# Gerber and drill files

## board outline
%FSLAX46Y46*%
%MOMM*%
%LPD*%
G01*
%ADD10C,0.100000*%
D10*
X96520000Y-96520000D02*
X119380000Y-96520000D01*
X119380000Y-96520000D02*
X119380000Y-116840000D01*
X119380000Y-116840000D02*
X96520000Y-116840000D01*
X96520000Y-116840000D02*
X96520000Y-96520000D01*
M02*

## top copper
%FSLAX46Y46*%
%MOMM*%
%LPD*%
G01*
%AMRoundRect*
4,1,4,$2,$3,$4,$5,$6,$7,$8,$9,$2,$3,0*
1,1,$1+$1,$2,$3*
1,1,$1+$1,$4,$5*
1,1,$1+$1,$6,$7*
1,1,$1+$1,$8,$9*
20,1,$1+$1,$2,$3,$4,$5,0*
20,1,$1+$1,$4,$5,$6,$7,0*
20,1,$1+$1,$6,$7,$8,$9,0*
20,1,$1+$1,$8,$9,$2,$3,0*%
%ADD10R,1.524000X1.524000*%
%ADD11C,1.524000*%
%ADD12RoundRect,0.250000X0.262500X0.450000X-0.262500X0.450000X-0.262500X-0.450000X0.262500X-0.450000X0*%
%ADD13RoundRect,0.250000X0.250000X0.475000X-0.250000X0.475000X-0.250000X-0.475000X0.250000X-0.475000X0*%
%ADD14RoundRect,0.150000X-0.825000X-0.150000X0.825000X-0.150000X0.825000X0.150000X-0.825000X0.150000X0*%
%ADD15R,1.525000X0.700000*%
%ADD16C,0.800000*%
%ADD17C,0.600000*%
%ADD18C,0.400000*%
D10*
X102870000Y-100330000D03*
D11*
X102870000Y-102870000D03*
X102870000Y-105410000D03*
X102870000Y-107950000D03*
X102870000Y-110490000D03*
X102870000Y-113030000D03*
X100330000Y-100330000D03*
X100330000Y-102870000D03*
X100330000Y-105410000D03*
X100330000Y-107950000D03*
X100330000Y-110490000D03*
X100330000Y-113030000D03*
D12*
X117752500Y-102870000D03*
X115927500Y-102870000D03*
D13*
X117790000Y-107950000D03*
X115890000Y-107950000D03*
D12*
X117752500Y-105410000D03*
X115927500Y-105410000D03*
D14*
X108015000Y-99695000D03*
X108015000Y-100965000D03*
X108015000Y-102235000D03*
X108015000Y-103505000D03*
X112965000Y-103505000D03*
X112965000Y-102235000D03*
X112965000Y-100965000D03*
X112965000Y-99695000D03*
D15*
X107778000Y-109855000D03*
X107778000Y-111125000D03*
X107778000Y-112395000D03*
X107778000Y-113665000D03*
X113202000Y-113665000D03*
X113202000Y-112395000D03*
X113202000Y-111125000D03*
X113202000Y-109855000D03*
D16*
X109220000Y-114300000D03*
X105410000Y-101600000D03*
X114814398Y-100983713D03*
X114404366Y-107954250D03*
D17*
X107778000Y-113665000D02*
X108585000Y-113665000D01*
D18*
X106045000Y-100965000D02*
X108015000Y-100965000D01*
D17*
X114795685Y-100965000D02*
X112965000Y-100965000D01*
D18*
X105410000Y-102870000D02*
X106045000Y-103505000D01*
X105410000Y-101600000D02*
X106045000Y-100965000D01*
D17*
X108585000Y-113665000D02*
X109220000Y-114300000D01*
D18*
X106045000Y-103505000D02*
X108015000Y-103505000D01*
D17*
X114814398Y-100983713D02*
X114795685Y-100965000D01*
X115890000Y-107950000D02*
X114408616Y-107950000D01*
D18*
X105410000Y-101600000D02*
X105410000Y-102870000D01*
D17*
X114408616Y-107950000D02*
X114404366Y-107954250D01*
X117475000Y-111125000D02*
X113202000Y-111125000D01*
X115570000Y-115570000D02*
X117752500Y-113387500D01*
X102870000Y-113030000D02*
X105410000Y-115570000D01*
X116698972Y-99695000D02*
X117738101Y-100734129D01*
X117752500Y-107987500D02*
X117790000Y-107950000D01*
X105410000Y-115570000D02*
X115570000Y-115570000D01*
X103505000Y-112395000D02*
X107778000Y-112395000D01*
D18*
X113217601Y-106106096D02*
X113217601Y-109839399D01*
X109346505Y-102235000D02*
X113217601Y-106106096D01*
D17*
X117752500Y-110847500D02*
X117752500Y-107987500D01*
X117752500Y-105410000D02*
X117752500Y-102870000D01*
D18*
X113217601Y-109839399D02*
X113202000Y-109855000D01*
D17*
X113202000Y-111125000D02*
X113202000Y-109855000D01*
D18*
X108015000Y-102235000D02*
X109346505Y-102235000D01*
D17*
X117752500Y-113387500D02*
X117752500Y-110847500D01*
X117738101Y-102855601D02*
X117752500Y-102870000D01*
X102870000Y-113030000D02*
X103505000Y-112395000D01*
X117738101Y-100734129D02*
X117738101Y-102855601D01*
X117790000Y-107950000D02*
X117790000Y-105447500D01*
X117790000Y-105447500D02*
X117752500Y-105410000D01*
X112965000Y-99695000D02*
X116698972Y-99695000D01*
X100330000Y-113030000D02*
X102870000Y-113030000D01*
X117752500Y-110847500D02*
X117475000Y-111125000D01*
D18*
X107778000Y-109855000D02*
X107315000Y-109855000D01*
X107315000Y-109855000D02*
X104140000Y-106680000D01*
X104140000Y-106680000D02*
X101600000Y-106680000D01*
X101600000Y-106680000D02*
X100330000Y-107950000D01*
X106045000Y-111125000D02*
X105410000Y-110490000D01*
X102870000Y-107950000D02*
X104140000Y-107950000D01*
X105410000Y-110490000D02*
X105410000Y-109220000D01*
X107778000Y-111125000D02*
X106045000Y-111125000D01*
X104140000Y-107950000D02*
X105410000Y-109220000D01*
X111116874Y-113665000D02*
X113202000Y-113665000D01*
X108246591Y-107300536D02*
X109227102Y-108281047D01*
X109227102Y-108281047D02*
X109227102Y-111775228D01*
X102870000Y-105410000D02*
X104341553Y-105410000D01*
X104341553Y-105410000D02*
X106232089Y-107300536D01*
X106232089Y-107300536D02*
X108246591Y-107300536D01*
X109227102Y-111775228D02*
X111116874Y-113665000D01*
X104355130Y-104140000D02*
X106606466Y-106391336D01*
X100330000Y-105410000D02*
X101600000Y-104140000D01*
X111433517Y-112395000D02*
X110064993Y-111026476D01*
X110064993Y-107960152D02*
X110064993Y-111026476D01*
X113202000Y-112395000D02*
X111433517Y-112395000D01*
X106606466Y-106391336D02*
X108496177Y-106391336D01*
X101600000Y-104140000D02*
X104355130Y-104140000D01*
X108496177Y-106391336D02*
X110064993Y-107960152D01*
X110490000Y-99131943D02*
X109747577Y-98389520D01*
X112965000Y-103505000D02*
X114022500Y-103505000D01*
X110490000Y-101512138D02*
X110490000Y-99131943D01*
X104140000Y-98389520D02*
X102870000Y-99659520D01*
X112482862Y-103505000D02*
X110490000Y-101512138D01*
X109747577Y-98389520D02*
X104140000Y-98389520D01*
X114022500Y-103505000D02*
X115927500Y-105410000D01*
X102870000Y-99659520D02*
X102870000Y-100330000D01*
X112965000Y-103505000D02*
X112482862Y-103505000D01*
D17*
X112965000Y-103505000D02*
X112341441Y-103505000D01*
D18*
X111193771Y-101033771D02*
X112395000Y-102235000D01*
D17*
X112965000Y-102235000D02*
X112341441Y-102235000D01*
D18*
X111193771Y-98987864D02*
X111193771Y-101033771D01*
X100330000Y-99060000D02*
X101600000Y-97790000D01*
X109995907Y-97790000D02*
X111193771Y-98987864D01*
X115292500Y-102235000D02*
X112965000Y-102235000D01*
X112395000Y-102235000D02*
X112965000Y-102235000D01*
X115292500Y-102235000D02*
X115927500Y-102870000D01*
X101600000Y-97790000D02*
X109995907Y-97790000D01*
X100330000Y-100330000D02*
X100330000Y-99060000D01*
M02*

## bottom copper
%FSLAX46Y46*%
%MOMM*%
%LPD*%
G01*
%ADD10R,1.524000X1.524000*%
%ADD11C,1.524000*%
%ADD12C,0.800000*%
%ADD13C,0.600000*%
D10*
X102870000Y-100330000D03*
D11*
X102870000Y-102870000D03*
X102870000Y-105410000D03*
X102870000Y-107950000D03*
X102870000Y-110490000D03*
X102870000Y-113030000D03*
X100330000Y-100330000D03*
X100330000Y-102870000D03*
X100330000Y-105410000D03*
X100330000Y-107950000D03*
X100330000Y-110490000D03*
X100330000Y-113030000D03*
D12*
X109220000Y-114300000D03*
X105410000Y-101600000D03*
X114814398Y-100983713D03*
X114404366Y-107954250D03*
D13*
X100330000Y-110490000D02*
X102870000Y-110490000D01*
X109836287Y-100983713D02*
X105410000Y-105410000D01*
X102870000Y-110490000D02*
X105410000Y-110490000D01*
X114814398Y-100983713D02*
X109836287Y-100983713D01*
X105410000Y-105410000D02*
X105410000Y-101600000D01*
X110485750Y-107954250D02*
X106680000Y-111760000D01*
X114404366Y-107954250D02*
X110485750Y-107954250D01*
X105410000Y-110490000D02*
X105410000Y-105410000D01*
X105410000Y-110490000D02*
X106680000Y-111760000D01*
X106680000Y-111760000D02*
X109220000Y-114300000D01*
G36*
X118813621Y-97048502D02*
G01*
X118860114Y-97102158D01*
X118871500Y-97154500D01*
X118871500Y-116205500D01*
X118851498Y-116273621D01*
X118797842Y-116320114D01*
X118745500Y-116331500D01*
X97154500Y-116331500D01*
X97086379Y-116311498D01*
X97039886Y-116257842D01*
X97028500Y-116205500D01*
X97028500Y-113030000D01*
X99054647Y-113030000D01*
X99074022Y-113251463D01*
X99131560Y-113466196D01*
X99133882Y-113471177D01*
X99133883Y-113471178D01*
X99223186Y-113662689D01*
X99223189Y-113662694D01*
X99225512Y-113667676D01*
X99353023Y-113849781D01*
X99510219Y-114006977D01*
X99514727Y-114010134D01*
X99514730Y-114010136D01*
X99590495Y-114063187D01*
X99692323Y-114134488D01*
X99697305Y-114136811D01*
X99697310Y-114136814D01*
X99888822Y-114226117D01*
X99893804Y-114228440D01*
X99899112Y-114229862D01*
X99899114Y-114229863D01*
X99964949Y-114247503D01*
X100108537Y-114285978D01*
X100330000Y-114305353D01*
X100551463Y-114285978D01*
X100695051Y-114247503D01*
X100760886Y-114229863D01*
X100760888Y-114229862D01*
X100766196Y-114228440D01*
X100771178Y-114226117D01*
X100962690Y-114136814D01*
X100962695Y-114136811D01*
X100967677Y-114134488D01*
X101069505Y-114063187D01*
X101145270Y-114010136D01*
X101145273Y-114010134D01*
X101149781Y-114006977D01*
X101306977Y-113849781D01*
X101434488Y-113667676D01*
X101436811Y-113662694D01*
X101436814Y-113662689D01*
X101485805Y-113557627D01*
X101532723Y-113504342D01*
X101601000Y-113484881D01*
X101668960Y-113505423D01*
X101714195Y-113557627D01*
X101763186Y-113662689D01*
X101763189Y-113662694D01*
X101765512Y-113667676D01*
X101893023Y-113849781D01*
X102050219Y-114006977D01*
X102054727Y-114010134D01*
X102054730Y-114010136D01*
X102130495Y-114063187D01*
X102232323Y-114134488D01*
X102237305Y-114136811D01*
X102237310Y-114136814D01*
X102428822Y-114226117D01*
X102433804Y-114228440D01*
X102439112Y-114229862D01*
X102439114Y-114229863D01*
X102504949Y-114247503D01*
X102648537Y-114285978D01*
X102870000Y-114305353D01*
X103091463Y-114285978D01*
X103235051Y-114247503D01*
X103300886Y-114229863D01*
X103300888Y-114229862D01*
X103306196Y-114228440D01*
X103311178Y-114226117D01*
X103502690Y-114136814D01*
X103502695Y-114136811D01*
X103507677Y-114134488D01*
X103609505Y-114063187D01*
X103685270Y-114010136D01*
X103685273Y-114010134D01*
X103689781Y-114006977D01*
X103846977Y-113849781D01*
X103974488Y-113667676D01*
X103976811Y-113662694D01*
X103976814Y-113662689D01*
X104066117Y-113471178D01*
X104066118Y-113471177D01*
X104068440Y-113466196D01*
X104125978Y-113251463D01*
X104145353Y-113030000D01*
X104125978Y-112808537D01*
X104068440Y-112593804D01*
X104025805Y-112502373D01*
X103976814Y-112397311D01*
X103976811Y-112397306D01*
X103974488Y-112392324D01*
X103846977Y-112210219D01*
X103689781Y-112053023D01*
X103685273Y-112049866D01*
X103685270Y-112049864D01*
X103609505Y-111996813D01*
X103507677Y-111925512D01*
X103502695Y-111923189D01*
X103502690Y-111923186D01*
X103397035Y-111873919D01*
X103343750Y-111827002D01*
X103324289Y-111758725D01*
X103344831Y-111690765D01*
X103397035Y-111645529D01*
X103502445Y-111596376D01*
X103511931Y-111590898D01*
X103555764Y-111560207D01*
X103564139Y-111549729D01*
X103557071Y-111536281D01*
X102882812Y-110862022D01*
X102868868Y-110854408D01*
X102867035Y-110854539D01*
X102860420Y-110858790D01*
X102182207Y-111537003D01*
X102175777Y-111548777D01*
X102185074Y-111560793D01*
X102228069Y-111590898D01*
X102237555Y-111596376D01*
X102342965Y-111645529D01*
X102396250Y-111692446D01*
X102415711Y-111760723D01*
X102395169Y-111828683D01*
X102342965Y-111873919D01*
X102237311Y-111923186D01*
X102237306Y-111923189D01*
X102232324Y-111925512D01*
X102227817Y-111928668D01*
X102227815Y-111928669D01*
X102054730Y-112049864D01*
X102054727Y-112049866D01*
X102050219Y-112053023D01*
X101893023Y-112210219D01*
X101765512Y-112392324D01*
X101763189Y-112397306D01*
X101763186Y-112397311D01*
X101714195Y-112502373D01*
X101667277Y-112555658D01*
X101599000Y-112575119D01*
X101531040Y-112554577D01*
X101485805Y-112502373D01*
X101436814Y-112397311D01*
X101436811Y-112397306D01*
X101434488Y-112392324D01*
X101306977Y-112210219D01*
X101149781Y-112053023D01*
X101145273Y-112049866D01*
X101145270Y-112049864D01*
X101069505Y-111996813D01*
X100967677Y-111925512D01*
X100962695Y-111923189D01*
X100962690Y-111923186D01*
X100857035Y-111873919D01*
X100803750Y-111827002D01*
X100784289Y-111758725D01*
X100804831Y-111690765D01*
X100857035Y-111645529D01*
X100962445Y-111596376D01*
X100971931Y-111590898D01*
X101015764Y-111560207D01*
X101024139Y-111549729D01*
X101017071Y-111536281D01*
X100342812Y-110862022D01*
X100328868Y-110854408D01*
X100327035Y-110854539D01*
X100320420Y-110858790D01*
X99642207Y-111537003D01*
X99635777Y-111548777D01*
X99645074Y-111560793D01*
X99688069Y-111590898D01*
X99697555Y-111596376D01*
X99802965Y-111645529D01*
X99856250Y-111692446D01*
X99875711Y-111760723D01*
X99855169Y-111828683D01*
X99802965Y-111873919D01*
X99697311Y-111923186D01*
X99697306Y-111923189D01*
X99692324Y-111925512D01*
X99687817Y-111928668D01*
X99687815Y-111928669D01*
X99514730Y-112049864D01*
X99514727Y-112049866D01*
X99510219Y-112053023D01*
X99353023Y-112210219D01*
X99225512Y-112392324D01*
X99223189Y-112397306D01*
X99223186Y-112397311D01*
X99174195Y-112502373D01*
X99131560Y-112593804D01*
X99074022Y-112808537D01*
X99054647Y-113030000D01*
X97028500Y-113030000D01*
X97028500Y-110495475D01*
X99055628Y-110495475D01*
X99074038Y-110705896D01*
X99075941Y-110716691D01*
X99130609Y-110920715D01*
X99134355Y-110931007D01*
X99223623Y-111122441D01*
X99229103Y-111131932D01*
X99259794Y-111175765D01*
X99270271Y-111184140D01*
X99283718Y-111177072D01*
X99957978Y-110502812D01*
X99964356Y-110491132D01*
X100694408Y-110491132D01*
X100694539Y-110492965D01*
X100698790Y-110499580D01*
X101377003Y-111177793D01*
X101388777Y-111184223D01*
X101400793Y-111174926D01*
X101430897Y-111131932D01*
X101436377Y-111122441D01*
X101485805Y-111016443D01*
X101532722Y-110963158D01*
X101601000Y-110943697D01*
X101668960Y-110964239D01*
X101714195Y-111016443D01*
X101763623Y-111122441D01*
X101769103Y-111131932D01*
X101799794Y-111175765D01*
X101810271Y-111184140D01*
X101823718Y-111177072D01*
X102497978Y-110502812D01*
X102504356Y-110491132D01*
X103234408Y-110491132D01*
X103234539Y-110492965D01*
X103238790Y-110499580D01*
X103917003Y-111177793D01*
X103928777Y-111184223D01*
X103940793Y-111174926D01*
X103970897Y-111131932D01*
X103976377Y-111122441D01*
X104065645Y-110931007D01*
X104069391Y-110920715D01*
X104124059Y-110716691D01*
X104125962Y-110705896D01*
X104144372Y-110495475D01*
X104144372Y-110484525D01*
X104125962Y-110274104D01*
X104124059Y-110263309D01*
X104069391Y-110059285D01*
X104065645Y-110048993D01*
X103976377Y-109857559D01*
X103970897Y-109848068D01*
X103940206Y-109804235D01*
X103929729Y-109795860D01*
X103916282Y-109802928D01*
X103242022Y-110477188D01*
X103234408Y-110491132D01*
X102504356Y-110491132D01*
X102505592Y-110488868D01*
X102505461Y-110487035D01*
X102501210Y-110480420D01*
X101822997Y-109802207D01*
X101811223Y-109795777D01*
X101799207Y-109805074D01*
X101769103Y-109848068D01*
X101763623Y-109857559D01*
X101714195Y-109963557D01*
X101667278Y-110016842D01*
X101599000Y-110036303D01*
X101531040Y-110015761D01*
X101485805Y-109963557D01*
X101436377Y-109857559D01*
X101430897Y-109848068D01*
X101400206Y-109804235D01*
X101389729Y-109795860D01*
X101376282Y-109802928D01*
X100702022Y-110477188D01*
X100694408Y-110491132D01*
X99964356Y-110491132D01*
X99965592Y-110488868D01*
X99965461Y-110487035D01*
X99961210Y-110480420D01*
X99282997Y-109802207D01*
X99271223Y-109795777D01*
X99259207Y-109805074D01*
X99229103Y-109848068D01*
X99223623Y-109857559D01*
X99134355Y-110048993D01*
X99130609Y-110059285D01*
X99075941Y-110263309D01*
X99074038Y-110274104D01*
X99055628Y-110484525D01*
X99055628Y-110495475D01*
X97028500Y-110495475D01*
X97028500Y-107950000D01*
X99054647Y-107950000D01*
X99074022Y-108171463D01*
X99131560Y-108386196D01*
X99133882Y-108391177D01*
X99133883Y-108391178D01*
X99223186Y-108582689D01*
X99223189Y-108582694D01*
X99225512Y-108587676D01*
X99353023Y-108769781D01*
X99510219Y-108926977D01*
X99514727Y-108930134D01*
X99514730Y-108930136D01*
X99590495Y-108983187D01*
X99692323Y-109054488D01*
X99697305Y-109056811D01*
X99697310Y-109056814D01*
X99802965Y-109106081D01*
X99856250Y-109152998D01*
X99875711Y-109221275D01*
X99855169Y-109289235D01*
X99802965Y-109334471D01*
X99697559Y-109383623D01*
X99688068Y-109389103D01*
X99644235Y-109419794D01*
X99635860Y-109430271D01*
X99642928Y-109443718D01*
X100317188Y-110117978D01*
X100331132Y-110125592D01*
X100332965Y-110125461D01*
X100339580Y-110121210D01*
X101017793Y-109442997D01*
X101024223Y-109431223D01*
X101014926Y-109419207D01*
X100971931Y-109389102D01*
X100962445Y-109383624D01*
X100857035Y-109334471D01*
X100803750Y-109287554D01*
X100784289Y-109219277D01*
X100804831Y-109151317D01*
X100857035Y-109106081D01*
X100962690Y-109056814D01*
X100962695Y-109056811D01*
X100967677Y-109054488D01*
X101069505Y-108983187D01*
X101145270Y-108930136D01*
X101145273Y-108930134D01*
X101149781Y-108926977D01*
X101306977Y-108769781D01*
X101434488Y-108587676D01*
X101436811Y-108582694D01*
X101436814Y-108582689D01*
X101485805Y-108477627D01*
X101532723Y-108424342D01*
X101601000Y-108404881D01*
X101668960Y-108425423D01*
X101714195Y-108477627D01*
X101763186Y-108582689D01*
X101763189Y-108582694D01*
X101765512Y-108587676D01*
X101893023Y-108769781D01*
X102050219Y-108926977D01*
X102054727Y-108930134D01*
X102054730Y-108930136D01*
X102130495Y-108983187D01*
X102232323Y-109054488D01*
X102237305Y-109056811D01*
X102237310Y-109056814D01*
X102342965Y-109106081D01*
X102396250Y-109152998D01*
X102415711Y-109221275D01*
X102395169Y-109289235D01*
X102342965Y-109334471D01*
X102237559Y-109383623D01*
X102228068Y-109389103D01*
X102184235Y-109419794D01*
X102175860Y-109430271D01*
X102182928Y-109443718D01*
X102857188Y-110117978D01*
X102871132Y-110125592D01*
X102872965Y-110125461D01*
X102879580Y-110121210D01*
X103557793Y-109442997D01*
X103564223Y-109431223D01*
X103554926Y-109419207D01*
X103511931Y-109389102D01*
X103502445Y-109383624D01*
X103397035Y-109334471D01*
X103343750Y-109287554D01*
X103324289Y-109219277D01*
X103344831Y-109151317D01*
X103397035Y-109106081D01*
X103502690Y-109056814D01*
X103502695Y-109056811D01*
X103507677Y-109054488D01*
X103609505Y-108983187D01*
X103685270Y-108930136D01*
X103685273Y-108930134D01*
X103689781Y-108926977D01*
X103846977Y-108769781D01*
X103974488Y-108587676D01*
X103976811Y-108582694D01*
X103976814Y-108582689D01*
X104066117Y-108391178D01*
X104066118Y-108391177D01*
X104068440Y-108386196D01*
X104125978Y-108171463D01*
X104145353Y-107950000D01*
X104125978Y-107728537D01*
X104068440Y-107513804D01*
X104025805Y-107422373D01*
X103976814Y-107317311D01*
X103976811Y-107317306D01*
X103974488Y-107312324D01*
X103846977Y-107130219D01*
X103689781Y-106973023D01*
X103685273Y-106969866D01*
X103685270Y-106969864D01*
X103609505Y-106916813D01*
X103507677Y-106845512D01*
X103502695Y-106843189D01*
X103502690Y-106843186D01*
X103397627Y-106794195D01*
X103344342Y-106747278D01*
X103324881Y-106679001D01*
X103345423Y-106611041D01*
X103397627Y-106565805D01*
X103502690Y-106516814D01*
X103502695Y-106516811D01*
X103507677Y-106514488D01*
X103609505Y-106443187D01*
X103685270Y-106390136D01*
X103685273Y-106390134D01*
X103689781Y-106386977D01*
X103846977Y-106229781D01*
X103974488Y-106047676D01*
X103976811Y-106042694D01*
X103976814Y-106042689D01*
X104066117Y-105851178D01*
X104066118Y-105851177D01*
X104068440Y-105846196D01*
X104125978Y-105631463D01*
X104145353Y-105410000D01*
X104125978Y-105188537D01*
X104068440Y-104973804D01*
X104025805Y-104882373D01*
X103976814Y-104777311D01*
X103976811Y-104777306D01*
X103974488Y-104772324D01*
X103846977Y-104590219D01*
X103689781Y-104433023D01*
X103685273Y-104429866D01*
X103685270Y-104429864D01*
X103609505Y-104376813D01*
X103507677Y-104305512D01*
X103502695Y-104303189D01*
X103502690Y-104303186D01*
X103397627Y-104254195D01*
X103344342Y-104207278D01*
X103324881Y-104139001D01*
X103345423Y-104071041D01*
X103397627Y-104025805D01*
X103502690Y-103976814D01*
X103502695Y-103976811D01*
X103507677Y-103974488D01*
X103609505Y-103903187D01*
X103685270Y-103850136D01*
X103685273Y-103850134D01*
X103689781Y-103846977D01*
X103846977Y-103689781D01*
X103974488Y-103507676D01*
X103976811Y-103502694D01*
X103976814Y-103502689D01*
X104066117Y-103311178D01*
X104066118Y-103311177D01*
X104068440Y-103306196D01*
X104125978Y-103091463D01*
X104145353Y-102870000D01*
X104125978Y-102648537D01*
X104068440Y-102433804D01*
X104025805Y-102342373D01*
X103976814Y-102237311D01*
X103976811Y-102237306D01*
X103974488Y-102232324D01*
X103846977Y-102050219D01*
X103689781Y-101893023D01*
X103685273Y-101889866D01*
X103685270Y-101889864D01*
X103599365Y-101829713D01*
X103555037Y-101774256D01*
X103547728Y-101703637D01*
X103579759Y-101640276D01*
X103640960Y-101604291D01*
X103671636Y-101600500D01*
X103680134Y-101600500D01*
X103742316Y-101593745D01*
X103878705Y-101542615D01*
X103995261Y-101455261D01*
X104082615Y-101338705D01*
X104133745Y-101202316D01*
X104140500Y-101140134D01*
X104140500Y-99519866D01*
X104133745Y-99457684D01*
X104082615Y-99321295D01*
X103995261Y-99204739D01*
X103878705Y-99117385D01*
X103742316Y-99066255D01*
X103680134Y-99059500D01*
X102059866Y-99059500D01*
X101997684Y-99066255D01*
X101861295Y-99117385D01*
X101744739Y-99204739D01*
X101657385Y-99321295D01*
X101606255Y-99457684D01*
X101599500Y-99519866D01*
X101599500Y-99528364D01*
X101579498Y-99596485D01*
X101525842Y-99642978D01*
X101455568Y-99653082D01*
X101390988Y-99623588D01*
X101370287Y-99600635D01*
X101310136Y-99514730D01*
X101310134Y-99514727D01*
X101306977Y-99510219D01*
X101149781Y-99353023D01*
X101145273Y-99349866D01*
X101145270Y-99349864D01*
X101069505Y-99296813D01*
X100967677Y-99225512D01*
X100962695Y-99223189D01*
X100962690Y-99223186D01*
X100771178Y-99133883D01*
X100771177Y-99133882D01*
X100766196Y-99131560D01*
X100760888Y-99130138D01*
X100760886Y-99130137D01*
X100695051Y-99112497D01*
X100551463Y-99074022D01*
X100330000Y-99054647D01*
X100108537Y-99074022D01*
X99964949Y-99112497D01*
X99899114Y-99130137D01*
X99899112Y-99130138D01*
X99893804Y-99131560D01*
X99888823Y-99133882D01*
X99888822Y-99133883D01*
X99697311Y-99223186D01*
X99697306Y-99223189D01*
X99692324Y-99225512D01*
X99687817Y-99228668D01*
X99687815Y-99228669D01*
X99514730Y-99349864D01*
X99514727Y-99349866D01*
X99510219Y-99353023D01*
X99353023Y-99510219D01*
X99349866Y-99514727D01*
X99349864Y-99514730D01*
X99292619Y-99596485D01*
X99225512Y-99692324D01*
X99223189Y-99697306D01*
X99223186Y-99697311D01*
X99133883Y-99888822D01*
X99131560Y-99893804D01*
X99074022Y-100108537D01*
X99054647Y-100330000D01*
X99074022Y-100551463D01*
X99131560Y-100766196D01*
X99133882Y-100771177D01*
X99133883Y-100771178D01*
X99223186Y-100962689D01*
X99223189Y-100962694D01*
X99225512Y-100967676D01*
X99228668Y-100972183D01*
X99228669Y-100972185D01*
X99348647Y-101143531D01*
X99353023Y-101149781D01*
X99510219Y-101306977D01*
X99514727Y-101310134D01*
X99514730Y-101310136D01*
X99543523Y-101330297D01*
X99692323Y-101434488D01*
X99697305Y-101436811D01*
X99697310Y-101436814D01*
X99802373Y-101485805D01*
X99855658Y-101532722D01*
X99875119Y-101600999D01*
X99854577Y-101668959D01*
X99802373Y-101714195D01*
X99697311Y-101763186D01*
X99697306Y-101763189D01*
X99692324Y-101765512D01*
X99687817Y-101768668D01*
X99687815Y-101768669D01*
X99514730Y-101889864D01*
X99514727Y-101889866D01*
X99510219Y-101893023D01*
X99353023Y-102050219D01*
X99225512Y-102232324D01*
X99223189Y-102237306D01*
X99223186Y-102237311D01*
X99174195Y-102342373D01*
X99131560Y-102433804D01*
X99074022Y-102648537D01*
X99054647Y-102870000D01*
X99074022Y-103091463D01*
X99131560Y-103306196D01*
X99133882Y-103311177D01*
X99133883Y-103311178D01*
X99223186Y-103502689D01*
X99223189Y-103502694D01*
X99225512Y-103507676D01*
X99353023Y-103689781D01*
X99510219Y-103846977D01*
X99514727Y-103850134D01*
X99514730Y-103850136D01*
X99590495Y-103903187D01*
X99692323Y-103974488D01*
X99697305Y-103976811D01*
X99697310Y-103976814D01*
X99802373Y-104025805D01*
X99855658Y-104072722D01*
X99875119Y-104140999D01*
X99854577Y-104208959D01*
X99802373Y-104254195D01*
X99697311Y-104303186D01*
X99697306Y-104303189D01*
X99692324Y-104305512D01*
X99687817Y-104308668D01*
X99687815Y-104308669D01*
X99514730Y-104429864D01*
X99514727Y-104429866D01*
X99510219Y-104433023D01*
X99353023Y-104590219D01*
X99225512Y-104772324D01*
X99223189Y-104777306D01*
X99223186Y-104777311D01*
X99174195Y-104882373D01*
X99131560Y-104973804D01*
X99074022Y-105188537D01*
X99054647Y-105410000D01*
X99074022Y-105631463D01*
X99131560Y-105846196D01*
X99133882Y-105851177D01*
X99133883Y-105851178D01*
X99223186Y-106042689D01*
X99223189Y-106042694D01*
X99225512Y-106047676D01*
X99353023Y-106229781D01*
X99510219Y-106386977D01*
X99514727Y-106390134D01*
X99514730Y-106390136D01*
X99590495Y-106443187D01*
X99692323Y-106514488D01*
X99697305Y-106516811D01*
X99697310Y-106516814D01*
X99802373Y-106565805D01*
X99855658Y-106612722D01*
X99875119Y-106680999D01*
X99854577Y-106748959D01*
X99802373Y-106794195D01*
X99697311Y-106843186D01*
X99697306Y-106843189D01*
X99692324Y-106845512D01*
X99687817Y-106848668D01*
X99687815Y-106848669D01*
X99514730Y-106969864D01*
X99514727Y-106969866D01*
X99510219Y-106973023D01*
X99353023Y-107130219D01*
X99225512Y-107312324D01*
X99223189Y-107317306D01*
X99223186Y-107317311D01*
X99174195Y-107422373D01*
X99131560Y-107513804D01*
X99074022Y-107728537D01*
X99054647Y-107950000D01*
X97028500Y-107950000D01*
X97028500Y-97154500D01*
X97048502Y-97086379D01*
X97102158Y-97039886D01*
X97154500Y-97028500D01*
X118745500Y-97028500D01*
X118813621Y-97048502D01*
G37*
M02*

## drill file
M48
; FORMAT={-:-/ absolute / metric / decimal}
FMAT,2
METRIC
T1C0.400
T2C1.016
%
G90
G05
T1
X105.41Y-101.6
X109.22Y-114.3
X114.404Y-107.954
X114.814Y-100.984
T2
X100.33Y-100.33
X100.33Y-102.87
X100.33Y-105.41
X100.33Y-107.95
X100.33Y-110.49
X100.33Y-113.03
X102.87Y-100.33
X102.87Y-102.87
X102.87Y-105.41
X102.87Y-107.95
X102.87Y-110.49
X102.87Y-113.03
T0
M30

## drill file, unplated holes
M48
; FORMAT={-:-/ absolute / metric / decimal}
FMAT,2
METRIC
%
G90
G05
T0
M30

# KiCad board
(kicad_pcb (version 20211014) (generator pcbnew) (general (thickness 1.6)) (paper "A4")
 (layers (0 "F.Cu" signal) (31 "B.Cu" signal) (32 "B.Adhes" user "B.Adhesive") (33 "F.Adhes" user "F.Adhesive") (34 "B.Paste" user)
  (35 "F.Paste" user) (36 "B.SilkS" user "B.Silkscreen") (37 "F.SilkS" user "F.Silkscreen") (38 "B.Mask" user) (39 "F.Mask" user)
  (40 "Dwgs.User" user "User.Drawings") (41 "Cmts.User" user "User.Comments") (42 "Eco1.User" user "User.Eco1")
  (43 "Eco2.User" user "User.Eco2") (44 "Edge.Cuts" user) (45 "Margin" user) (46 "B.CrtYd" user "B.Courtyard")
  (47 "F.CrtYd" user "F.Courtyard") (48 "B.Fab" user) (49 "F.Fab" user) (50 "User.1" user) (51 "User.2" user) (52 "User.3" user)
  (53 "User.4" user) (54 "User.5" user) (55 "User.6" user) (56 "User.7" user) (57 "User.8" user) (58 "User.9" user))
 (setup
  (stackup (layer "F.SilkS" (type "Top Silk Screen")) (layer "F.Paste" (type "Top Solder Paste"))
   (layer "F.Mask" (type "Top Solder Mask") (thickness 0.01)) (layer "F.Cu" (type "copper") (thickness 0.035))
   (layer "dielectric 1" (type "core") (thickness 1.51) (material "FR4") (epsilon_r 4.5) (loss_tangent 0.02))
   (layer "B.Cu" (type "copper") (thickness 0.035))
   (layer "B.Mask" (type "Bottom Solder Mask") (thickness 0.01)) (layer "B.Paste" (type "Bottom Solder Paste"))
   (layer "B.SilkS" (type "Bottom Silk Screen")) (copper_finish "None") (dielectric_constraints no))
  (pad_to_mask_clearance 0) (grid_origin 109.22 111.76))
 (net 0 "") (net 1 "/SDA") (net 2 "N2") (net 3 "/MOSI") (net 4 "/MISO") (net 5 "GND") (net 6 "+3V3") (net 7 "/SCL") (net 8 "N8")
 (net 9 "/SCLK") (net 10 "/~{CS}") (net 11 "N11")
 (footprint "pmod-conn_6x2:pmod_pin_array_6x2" (layer "F.Cu") (at 101.6 106.68)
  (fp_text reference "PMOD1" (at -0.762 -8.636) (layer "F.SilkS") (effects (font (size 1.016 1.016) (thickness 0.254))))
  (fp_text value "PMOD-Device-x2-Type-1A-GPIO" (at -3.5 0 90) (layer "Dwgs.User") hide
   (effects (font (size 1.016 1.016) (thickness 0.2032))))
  (pad "1" thru_hole rect locked (at 1.27 -6.35) (size 1.524 1.524) (drill 1.016) (layers *.Cu *.Mask "F.SilkS") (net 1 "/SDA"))
  (pad "2" thru_hole circle locked (at 1.27 -3.81 270) (size 1.524 1.524) (drill 1.016) (layers *.Cu *.Mask "F.SilkS") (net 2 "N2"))
  (pad "3" thru_hole circle locked (at 1.27 -1.27 270) (size 1.524 1.524) (drill 1.016) (layers *.Cu *.Mask "F.SilkS") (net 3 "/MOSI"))
  (pad "4" thru_hole circle locked (at 1.27 1.27 270) (size 1.524 1.524) (drill 1.016) (layers *.Cu *.Mask "F.SilkS") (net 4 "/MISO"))
  (pad "5" thru_hole circle locked (at 1.27 3.81 270) (size 1.524 1.524) (drill 1.016) (layers *.Cu *.Mask "F.SilkS") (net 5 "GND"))
  (pad "6" thru_hole circle locked (at 1.27 6.35 270) (size 1.524 1.524) (drill 1.016) (layers *.Cu *.Mask "F.SilkS") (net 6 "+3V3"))
  (pad "7" thru_hole circle locked (at -1.27 -6.35 270) (size 1.524 1.524) (drill 1.016) (layers *.Cu *.Mask "F.SilkS") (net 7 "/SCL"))
  (pad "8" thru_hole circle locked (at -1.27 -3.81 270) (size 1.524 1.524) (drill 1.016) (layers *.Cu *.Mask "F.SilkS") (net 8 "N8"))
  (pad "9" thru_hole circle locked (at -1.27 -1.27 270) (size 1.524 1.524) (drill 1.016) (layers *.Cu *.Mask "F.SilkS") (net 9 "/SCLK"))
  (pad "10" thru_hole circle locked (at -1.27 1.27 270) (size 1.524 1.524) (drill 1.016) (layers *.Cu *.Mask "F.SilkS") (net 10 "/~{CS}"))
  (pad "11" thru_hole circle locked (at -1.27 3.81 270) (size 1.524 1.524) (drill 1.016) (layers *.Cu *.Mask "F.SilkS") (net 5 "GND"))
  (pad "12" thru_hole circle locked (at -1.27 6.35 270) (size 1.524 1.524) (drill 1.016) (layers *.Cu *.Mask "F.SilkS") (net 6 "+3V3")))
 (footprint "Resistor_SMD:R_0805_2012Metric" (layer "F.Cu") (at 116.84 102.87 180)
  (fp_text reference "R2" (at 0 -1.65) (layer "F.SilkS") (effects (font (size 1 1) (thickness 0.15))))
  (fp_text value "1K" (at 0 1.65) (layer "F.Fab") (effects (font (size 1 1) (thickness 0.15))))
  (pad "1" smd roundrect (at -0.9125 0 180) (size 1.025 1.4) (layers "F.Cu" "F.Paste" "F.Mask") (roundrect_rratio 0.243902439)
   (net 6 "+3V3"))
  (pad "2" smd roundrect (at 0.9125 0 180) (size 1.025 1.4) (layers "F.Cu" "F.Paste" "F.Mask") (roundrect_rratio 0.243902439) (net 7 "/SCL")))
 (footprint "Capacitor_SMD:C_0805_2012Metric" (layer "F.Cu") (at 116.84 107.95 180)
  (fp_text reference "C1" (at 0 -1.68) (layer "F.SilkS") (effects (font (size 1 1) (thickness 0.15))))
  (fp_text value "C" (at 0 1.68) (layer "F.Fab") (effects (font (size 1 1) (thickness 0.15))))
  (pad "1" smd roundrect (at -0.95 0 180) (size 1 1.45) (layers "F.Cu" "F.Paste" "F.Mask") (roundrect_rratio 0.25) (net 6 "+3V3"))
  (pad "2" smd roundrect (at 0.95 0 180) (size 1 1.45) (layers "F.Cu" "F.Paste" "F.Mask") (roundrect_rratio 0.25) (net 5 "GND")))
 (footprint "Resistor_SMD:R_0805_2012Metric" (layer "F.Cu") (at 116.84 105.41 180)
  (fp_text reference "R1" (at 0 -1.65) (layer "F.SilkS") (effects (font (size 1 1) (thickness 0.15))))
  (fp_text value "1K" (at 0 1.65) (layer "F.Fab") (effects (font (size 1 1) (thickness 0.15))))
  (pad "1" smd roundrect (at -0.9125 0 180) (size 1.025 1.4) (layers "F.Cu" "F.Paste" "F.Mask") (roundrect_rratio 0.243902439)
   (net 6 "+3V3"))
  (pad "2" smd roundrect (at 0.9125 0 180) (size 1.025 1.4) (layers "F.Cu" "F.Paste" "F.Mask") (roundrect_rratio 0.243902439) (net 1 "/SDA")))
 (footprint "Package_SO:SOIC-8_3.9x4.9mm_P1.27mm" (layer "F.Cu") (at 110.49 101.6)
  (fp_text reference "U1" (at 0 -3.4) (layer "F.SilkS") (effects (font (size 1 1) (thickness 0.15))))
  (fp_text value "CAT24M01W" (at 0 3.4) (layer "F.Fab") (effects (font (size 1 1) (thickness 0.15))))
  (pad "1" smd roundrect (at -2.475 -1.905) (size 1.95 0.6) (layers "F.Cu" "F.Paste" "F.Mask") (roundrect_rratio 0.25) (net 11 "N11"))
  (pad "2" smd roundrect (at -2.475 -0.635) (size 1.95 0.6) (layers "F.Cu" "F.Paste" "F.Mask") (roundrect_rratio 0.25) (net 5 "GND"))
  (pad "3" smd roundrect (at -2.475 0.635) (size 1.95 0.6) (layers "F.Cu" "F.Paste" "F.Mask") (roundrect_rratio 0.25) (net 6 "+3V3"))
  (pad "4" smd roundrect (at -2.475 1.905) (size 1.95 0.6) (layers "F.Cu" "F.Paste" "F.Mask") (roundrect_rratio 0.25) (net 5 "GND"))
  (pad "5" smd roundrect (at 2.475 1.905) (size 1.95 0.6) (layers "F.Cu" "F.Paste" "F.Mask") (roundrect_rratio 0.25) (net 1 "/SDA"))
  (pad "6" smd roundrect (at 2.475 0.635) (size 1.95 0.6) (layers "F.Cu" "F.Paste" "F.Mask") (roundrect_rratio 0.25) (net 7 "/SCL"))
  (pad "7" smd roundrect (at 2.475 -0.635) (size 1.95 0.6) (layers "F.Cu" "F.Paste" "F.Mask") (roundrect_rratio 0.25) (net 5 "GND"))
  (pad "8" smd roundrect (at 2.475 -1.905) (size 1.95 0.6) (layers "F.Cu" "F.Paste" "F.Mask") (roundrect_rratio 0.25) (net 6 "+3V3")))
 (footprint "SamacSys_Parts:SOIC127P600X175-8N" (layer "F.Cu") (at 110.49 111.76)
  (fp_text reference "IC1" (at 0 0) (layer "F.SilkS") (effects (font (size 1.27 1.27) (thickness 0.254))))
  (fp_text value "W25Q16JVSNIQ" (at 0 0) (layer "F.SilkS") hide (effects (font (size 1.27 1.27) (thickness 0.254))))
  (pad "1" smd rect locked (at -2.712 -1.905 90) (size 0.7 1.525) (layers "F.Cu" "F.Paste" "F.Mask") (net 10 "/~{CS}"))
  (pad "2" smd rect locked (at -2.712 -0.635 90) (size 0.7 1.525) (layers "F.Cu" "F.Paste" "F.Mask") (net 4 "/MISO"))
  (pad "3" smd rect locked (at -2.712 0.635 90) (size 0.7 1.525) (layers "F.Cu" "F.Paste" "F.Mask") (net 6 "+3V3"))
  (pad "4" smd rect locked (at -2.712 1.905 90) (size 0.7 1.525) (layers "F.Cu" "F.Paste" "F.Mask") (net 5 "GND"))
  (pad "5" smd rect locked (at 2.712 1.905 90) (size 0.7 1.525) (layers "F.Cu" "F.Paste" "F.Mask") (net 3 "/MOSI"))
  (pad "6" smd rect locked (at 2.712 0.635 90) (size 0.7 1.525) (layers "F.Cu" "F.Paste" "F.Mask") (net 9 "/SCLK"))
  (pad "7" smd rect locked (at 2.712 -0.635 90) (size 0.7 1.525) (layers "F.Cu" "F.Paste" "F.Mask") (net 6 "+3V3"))
  (pad "8" smd rect locked (at 2.712 -1.905 90) (size 0.7 1.525) (layers "F.Cu" "F.Paste" "F.Mask") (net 6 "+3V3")))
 (gr_rect (start 96.52 96.52) (end 119.38 116.84) (layer "Edge.Cuts") (width 0.1) (fill none))
 (segment (start 107.778 113.665) (end 108.585 113.665) (width 0.6) (layer "F.Cu") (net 5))
 (segment (start 106.045 100.965) (end 108.015 100.965) (width 0.4) (layer "F.Cu") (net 5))
 (segment (start 114.795685 100.965) (end 112.965 100.965) (width 0.6) (layer "F.Cu") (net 5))
 (segment (start 105.41 102.87) (end 106.045 103.505) (width 0.4) (layer "F.Cu") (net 5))
 (segment (start 105.41 101.6) (end 106.045 100.965) (width 0.4) (layer "F.Cu") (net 5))
 (segment (start 108.585 113.665) (end 109.22 114.3) (width 0.6) (layer "F.Cu") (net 5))
 (segment (start 106.045 103.505) (end 108.015 103.505) (width 0.4) (layer "F.Cu") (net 5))
 (segment (start 114.814398 100.983713) (end 114.795685 100.965) (width 0.6) (layer "F.Cu") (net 5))
 (segment (start 115.89 107.95) (end 114.408616 107.95) (width 0.6) (layer "F.Cu") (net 5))
 (segment (start 105.41 101.6) (end 105.41 102.87) (width 0.4) (layer "F.Cu") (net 5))
 (segment (start 114.408616 107.95) (end 114.404366 107.95425) (width 0.6) (layer "F.Cu") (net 5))
 (via (at 109.22 114.3) (size 0.8) (drill 0.4) (layers "F.Cu" "B.Cu") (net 5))
 (via (at 105.41 101.6) (size 0.8) (drill 0.4) (layers "F.Cu" "B.Cu") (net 5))
 (via (at 114.814398 100.983713) (size 0.8) (drill 0.4) (layers "F.Cu" "B.Cu") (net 5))
 (via (at 114.404366 107.95425) (size 0.8) (drill 0.4) (layers "F.Cu" "B.Cu") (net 5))
 (segment (start 100.33 110.49) (end 102.87 110.49) (width 0.6) (layer "B.Cu") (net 5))
 (segment (start 109.836287 100.983713) (end 105.41 105.41) (width 0.6) (layer "B.Cu") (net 5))
 (segment (start 102.87 110.49) (end 105.41 110.49) (width 0.6) (layer "B.Cu") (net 5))
 (segment (start 114.814398 100.983713) (end 109.836287 100.983713) (width 0.6) (layer "B.Cu") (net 5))
 (segment (start 105.41 105.41) (end 105.41 101.6) (width 0.6) (layer "B.Cu") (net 5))
 (segment (start 110.48575 107.95425) (end 106.68 111.76) (width 0.6) (layer "B.Cu") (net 5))
 (segment (start 114.404366 107.95425) (end 110.48575 107.95425) (width 0.6) (layer "B.Cu") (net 5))
 (segment (start 105.41 110.49) (end 105.41 105.41) (width 0.6) (layer "B.Cu") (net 5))
 (segment (start 105.41 110.49) (end 106.68 111.76) (width 0.6) (layer "B.Cu") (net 5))
 (segment (start 106.68 111.76) (end 109.22 114.3) (width 0.6) (layer "B.Cu") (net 5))
 (segment (start 117.475 111.125) (end 113.202 111.125) (width 0.6) (layer "F.Cu") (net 6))
 (segment (start 115.57 115.57) (end 117.7525 113.3875) (width 0.6) (layer "F.Cu") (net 6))
 (segment (start 102.87 113.03) (end 105.41 115.57) (width 0.6) (layer "F.Cu") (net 6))
 (segment (start 116.698972 99.695) (end 117.738101 100.734129) (width 0.6) (layer "F.Cu") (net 6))
 (segment (start 117.7525 107.9875) (end 117.79 107.95) (width 0.6) (layer "F.Cu") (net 6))
 (segment (start 105.41 115.57) (end 115.57 115.57) (width 0.6) (layer "F.Cu") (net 6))
 (segment (start 103.505 112.395) (end 107.778 112.395) (width 0.6) (layer "F.Cu") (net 6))
 (segment (start 113.217601 106.106096) (end 113.217601 109.839399) (width 0.4) (layer "F.Cu") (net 6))
 (segment (start 109.346505 102.235) (end 113.217601 106.106096) (width 0.4) (layer "F.Cu") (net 6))
 (segment (start 117.7525 110.8475) (end 117.7525 107.9875) (width 0.6) (layer "F.Cu") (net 6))
 (segment (start 117.7525 105.41) (end 117.7525 102.87) (width 0.6) (layer "F.Cu") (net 6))
 (segment (start 113.217601 109.839399) (end 113.202 109.855) (width 0.4) (layer "F.Cu") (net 6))
 (segment (start 113.202 111.125) (end 113.202 109.855) (width 0.6) (layer "F.Cu") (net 6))
 (segment (start 108.015 102.235) (end 109.346505 102.235) (width 0.4) (layer "F.Cu") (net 6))
 (segment (start 117.7525 113.3875) (end 117.7525 110.8475) (width 0.6) (layer "F.Cu") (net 6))
 (segment (start 117.738101 102.855601) (end 117.7525 102.87) (width 0.6) (layer "F.Cu") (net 6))
 (segment (start 102.87 113.03) (end 103.505 112.395) (width 0.6) (layer "F.Cu") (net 6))
 (segment (start 117.738101 100.734129) (end 117.738101 102.855601) (width 0.6) (layer "F.Cu") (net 6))
 (segment (start 117.79 107.95) (end 117.79 105.4475) (width 0.6) (layer "F.Cu") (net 6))
 (segment (start 117.79 105.4475) (end 117.7525 105.41) (width 0.6) (layer "F.Cu") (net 6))
 (segment (start 112.965 99.695) (end 116.698972 99.695) (width 0.6) (layer "F.Cu") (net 6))
 (segment (start 100.33 113.03) (end 102.87 113.03) (width 0.6) (layer "F.Cu") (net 6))
 (segment (start 117.7525 110.8475) (end 117.475 111.125) (width 0.6) (layer "F.Cu") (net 6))
 (segment (start 107.778 109.855) (end 107.315 109.855) (width 0.4) (layer "F.Cu") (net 10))
 (segment (start 107.315 109.855) (end 104.14 106.68) (width 0.4) (layer "F.Cu") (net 10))
 (segment (start 104.14 106.68) (end 101.6 106.68) (width 0.4) (layer "F.Cu") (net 10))
 (segment (start 101.6 106.68) (end 100.33 107.95) (width 0.4) (layer "F.Cu") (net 10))
 (segment (start 106.045 111.125) (end 105.41 110.49) (width 0.4) (layer "F.Cu") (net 4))
 (segment (start 102.87 107.95) (end 104.14 107.95) (width 0.4) (layer "F.Cu") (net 4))
 (segment (start 105.41 110.49) (end 105.41 109.22) (width 0.4) (layer "F.Cu") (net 4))
 (segment (start 107.778 111.125) (end 106.045 111.125) (width 0.4) (layer "F.Cu") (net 4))
 (segment (start 104.14 107.95) (end 105.41 109.22) (width 0.4) (layer "F.Cu") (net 4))
 (segment (start 111.116874 113.665) (end 113.202 113.665) (width 0.4) (layer "F.Cu") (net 3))
 (segment (start 108.246591 107.300536) (end 109.227102 108.281047) (width 0.4) (layer "F.Cu") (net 3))
 (segment (start 109.227102 108.281047) (end 109.227102 111.775228) (width 0.4) (layer "F.Cu") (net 3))
 (segment (start 102.87 105.41) (end 104.341553 105.41) (width 0.4) (layer "F.Cu") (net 3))
 (segment (start 104.341553 105.41) (end 106.232089 107.300536) (width 0.4) (layer "F.Cu") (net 3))
 (segment (start 106.232089 107.300536) (end 108.246591 107.300536) (width 0.4) (layer "F.Cu") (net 3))
 (segment (start 109.227102 111.775228) (end 111.116874 113.665) (width 0.4) (layer "F.Cu") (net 3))
 (segment (start 104.35513 104.14) (end 106.606466 106.391336) (width 0.4) (layer "F.Cu") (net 9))
 (segment (start 100.33 105.41) (end 101.6 104.14) (width 0.4) (layer "F.Cu") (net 9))
 (segment (start 111.433517 112.395) (end 110.064993 111.026476) (width 0.4) (layer "F.Cu") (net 9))
 (segment (start 110.064993 107.960152) (end 110.064993 111.026476) (width 0.4) (layer "F.Cu") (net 9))
 (segment (start 113.202 112.395) (end 111.433517 112.395) (width 0.4) (layer "F.Cu") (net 9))
 (segment (start 106.606466 106.391336) (end 108.496177 106.391336) (width 0.4) (layer "F.Cu") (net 9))
 (segment (start 101.6 104.14) (end 104.35513 104.14) (width 0.4) (layer "F.Cu") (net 9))
 (segment (start 108.496177 106.391336) (end 110.064993 107.960152) (width 0.4) (layer "F.Cu") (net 9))
 (segment (start 110.49 99.131943) (end 109.747577 98.38952) (width 0.4) (layer "F.Cu") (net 1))
 (segment (start 112.965 103.505) (end 114.0225 103.505) (width 0.4) (layer "F.Cu") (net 1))
 (segment (start 110.49 101.512138) (end 110.49 99.131943) (width 0.4) (layer "F.Cu") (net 1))
 (segment (start 104.14 98.38952) (end 102.87 99.65952) (width 0.4) (layer "F.Cu") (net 1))
 (segment (start 112.482862 103.505) (end 110.49 101.512138) (width 0.4) (layer "F.Cu") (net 1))
 (segment (start 109.747577 98.38952) (end 104.14 98.38952) (width 0.4) (layer "F.Cu") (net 1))
 (segment (start 114.0225 103.505) (end 115.9275 105.41) (width 0.4) (layer "F.Cu") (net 1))
 (segment (start 102.87 99.65952) (end 102.87 100.33) (width 0.4) (layer "F.Cu") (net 1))
 (segment (start 112.965 103.505) (end 112.482862 103.505) (width 0.4) (layer "F.Cu") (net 1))
 (segment (start 112.965 103.505) (end 112.341441 103.505) (width 0.6) (layer "F.Cu") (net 1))
 (segment (start 111.193771 101.033771) (end 112.395 102.235) (width 0.4) (layer "F.Cu") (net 7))
 (segment (start 112.965 102.235) (end 112.341441 102.235) (width 0.6) (layer "F.Cu") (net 7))
 (segment (start 111.193771 98.987864) (end 111.193771 101.033771) (width 0.4) (layer "F.Cu") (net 7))
 (segment (start 100.33 99.06) (end 101.6 97.79) (width 0.4) (layer "F.Cu") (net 7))
 (segment (start 109.995907 97.79) (end 111.193771 98.987864) (width 0.4) (layer "F.Cu") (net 7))
 (segment (start 115.2925 102.235) (end 112.965 102.235) (width 0.4) (layer "F.Cu") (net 7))
 (segment (start 112.395 102.235) (end 112.965 102.235) (width 0.4) (layer "F.Cu") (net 7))
 (segment (start 115.2925 102.235) (end 115.9275 102.87) (width 0.4) (layer "F.Cu") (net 7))
 (segment (start 101.6 97.79) (end 109.995907 97.79) (width 0.4) (layer "F.Cu") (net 7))
 (segment (start 100.33 100.33) (end 100.33 99.06) (width 0.4) (layer "F.Cu") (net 7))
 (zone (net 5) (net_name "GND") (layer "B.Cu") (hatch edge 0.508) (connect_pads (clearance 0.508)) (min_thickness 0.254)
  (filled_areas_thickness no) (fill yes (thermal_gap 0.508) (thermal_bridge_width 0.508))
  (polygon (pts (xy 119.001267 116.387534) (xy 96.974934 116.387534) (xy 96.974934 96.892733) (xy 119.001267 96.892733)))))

